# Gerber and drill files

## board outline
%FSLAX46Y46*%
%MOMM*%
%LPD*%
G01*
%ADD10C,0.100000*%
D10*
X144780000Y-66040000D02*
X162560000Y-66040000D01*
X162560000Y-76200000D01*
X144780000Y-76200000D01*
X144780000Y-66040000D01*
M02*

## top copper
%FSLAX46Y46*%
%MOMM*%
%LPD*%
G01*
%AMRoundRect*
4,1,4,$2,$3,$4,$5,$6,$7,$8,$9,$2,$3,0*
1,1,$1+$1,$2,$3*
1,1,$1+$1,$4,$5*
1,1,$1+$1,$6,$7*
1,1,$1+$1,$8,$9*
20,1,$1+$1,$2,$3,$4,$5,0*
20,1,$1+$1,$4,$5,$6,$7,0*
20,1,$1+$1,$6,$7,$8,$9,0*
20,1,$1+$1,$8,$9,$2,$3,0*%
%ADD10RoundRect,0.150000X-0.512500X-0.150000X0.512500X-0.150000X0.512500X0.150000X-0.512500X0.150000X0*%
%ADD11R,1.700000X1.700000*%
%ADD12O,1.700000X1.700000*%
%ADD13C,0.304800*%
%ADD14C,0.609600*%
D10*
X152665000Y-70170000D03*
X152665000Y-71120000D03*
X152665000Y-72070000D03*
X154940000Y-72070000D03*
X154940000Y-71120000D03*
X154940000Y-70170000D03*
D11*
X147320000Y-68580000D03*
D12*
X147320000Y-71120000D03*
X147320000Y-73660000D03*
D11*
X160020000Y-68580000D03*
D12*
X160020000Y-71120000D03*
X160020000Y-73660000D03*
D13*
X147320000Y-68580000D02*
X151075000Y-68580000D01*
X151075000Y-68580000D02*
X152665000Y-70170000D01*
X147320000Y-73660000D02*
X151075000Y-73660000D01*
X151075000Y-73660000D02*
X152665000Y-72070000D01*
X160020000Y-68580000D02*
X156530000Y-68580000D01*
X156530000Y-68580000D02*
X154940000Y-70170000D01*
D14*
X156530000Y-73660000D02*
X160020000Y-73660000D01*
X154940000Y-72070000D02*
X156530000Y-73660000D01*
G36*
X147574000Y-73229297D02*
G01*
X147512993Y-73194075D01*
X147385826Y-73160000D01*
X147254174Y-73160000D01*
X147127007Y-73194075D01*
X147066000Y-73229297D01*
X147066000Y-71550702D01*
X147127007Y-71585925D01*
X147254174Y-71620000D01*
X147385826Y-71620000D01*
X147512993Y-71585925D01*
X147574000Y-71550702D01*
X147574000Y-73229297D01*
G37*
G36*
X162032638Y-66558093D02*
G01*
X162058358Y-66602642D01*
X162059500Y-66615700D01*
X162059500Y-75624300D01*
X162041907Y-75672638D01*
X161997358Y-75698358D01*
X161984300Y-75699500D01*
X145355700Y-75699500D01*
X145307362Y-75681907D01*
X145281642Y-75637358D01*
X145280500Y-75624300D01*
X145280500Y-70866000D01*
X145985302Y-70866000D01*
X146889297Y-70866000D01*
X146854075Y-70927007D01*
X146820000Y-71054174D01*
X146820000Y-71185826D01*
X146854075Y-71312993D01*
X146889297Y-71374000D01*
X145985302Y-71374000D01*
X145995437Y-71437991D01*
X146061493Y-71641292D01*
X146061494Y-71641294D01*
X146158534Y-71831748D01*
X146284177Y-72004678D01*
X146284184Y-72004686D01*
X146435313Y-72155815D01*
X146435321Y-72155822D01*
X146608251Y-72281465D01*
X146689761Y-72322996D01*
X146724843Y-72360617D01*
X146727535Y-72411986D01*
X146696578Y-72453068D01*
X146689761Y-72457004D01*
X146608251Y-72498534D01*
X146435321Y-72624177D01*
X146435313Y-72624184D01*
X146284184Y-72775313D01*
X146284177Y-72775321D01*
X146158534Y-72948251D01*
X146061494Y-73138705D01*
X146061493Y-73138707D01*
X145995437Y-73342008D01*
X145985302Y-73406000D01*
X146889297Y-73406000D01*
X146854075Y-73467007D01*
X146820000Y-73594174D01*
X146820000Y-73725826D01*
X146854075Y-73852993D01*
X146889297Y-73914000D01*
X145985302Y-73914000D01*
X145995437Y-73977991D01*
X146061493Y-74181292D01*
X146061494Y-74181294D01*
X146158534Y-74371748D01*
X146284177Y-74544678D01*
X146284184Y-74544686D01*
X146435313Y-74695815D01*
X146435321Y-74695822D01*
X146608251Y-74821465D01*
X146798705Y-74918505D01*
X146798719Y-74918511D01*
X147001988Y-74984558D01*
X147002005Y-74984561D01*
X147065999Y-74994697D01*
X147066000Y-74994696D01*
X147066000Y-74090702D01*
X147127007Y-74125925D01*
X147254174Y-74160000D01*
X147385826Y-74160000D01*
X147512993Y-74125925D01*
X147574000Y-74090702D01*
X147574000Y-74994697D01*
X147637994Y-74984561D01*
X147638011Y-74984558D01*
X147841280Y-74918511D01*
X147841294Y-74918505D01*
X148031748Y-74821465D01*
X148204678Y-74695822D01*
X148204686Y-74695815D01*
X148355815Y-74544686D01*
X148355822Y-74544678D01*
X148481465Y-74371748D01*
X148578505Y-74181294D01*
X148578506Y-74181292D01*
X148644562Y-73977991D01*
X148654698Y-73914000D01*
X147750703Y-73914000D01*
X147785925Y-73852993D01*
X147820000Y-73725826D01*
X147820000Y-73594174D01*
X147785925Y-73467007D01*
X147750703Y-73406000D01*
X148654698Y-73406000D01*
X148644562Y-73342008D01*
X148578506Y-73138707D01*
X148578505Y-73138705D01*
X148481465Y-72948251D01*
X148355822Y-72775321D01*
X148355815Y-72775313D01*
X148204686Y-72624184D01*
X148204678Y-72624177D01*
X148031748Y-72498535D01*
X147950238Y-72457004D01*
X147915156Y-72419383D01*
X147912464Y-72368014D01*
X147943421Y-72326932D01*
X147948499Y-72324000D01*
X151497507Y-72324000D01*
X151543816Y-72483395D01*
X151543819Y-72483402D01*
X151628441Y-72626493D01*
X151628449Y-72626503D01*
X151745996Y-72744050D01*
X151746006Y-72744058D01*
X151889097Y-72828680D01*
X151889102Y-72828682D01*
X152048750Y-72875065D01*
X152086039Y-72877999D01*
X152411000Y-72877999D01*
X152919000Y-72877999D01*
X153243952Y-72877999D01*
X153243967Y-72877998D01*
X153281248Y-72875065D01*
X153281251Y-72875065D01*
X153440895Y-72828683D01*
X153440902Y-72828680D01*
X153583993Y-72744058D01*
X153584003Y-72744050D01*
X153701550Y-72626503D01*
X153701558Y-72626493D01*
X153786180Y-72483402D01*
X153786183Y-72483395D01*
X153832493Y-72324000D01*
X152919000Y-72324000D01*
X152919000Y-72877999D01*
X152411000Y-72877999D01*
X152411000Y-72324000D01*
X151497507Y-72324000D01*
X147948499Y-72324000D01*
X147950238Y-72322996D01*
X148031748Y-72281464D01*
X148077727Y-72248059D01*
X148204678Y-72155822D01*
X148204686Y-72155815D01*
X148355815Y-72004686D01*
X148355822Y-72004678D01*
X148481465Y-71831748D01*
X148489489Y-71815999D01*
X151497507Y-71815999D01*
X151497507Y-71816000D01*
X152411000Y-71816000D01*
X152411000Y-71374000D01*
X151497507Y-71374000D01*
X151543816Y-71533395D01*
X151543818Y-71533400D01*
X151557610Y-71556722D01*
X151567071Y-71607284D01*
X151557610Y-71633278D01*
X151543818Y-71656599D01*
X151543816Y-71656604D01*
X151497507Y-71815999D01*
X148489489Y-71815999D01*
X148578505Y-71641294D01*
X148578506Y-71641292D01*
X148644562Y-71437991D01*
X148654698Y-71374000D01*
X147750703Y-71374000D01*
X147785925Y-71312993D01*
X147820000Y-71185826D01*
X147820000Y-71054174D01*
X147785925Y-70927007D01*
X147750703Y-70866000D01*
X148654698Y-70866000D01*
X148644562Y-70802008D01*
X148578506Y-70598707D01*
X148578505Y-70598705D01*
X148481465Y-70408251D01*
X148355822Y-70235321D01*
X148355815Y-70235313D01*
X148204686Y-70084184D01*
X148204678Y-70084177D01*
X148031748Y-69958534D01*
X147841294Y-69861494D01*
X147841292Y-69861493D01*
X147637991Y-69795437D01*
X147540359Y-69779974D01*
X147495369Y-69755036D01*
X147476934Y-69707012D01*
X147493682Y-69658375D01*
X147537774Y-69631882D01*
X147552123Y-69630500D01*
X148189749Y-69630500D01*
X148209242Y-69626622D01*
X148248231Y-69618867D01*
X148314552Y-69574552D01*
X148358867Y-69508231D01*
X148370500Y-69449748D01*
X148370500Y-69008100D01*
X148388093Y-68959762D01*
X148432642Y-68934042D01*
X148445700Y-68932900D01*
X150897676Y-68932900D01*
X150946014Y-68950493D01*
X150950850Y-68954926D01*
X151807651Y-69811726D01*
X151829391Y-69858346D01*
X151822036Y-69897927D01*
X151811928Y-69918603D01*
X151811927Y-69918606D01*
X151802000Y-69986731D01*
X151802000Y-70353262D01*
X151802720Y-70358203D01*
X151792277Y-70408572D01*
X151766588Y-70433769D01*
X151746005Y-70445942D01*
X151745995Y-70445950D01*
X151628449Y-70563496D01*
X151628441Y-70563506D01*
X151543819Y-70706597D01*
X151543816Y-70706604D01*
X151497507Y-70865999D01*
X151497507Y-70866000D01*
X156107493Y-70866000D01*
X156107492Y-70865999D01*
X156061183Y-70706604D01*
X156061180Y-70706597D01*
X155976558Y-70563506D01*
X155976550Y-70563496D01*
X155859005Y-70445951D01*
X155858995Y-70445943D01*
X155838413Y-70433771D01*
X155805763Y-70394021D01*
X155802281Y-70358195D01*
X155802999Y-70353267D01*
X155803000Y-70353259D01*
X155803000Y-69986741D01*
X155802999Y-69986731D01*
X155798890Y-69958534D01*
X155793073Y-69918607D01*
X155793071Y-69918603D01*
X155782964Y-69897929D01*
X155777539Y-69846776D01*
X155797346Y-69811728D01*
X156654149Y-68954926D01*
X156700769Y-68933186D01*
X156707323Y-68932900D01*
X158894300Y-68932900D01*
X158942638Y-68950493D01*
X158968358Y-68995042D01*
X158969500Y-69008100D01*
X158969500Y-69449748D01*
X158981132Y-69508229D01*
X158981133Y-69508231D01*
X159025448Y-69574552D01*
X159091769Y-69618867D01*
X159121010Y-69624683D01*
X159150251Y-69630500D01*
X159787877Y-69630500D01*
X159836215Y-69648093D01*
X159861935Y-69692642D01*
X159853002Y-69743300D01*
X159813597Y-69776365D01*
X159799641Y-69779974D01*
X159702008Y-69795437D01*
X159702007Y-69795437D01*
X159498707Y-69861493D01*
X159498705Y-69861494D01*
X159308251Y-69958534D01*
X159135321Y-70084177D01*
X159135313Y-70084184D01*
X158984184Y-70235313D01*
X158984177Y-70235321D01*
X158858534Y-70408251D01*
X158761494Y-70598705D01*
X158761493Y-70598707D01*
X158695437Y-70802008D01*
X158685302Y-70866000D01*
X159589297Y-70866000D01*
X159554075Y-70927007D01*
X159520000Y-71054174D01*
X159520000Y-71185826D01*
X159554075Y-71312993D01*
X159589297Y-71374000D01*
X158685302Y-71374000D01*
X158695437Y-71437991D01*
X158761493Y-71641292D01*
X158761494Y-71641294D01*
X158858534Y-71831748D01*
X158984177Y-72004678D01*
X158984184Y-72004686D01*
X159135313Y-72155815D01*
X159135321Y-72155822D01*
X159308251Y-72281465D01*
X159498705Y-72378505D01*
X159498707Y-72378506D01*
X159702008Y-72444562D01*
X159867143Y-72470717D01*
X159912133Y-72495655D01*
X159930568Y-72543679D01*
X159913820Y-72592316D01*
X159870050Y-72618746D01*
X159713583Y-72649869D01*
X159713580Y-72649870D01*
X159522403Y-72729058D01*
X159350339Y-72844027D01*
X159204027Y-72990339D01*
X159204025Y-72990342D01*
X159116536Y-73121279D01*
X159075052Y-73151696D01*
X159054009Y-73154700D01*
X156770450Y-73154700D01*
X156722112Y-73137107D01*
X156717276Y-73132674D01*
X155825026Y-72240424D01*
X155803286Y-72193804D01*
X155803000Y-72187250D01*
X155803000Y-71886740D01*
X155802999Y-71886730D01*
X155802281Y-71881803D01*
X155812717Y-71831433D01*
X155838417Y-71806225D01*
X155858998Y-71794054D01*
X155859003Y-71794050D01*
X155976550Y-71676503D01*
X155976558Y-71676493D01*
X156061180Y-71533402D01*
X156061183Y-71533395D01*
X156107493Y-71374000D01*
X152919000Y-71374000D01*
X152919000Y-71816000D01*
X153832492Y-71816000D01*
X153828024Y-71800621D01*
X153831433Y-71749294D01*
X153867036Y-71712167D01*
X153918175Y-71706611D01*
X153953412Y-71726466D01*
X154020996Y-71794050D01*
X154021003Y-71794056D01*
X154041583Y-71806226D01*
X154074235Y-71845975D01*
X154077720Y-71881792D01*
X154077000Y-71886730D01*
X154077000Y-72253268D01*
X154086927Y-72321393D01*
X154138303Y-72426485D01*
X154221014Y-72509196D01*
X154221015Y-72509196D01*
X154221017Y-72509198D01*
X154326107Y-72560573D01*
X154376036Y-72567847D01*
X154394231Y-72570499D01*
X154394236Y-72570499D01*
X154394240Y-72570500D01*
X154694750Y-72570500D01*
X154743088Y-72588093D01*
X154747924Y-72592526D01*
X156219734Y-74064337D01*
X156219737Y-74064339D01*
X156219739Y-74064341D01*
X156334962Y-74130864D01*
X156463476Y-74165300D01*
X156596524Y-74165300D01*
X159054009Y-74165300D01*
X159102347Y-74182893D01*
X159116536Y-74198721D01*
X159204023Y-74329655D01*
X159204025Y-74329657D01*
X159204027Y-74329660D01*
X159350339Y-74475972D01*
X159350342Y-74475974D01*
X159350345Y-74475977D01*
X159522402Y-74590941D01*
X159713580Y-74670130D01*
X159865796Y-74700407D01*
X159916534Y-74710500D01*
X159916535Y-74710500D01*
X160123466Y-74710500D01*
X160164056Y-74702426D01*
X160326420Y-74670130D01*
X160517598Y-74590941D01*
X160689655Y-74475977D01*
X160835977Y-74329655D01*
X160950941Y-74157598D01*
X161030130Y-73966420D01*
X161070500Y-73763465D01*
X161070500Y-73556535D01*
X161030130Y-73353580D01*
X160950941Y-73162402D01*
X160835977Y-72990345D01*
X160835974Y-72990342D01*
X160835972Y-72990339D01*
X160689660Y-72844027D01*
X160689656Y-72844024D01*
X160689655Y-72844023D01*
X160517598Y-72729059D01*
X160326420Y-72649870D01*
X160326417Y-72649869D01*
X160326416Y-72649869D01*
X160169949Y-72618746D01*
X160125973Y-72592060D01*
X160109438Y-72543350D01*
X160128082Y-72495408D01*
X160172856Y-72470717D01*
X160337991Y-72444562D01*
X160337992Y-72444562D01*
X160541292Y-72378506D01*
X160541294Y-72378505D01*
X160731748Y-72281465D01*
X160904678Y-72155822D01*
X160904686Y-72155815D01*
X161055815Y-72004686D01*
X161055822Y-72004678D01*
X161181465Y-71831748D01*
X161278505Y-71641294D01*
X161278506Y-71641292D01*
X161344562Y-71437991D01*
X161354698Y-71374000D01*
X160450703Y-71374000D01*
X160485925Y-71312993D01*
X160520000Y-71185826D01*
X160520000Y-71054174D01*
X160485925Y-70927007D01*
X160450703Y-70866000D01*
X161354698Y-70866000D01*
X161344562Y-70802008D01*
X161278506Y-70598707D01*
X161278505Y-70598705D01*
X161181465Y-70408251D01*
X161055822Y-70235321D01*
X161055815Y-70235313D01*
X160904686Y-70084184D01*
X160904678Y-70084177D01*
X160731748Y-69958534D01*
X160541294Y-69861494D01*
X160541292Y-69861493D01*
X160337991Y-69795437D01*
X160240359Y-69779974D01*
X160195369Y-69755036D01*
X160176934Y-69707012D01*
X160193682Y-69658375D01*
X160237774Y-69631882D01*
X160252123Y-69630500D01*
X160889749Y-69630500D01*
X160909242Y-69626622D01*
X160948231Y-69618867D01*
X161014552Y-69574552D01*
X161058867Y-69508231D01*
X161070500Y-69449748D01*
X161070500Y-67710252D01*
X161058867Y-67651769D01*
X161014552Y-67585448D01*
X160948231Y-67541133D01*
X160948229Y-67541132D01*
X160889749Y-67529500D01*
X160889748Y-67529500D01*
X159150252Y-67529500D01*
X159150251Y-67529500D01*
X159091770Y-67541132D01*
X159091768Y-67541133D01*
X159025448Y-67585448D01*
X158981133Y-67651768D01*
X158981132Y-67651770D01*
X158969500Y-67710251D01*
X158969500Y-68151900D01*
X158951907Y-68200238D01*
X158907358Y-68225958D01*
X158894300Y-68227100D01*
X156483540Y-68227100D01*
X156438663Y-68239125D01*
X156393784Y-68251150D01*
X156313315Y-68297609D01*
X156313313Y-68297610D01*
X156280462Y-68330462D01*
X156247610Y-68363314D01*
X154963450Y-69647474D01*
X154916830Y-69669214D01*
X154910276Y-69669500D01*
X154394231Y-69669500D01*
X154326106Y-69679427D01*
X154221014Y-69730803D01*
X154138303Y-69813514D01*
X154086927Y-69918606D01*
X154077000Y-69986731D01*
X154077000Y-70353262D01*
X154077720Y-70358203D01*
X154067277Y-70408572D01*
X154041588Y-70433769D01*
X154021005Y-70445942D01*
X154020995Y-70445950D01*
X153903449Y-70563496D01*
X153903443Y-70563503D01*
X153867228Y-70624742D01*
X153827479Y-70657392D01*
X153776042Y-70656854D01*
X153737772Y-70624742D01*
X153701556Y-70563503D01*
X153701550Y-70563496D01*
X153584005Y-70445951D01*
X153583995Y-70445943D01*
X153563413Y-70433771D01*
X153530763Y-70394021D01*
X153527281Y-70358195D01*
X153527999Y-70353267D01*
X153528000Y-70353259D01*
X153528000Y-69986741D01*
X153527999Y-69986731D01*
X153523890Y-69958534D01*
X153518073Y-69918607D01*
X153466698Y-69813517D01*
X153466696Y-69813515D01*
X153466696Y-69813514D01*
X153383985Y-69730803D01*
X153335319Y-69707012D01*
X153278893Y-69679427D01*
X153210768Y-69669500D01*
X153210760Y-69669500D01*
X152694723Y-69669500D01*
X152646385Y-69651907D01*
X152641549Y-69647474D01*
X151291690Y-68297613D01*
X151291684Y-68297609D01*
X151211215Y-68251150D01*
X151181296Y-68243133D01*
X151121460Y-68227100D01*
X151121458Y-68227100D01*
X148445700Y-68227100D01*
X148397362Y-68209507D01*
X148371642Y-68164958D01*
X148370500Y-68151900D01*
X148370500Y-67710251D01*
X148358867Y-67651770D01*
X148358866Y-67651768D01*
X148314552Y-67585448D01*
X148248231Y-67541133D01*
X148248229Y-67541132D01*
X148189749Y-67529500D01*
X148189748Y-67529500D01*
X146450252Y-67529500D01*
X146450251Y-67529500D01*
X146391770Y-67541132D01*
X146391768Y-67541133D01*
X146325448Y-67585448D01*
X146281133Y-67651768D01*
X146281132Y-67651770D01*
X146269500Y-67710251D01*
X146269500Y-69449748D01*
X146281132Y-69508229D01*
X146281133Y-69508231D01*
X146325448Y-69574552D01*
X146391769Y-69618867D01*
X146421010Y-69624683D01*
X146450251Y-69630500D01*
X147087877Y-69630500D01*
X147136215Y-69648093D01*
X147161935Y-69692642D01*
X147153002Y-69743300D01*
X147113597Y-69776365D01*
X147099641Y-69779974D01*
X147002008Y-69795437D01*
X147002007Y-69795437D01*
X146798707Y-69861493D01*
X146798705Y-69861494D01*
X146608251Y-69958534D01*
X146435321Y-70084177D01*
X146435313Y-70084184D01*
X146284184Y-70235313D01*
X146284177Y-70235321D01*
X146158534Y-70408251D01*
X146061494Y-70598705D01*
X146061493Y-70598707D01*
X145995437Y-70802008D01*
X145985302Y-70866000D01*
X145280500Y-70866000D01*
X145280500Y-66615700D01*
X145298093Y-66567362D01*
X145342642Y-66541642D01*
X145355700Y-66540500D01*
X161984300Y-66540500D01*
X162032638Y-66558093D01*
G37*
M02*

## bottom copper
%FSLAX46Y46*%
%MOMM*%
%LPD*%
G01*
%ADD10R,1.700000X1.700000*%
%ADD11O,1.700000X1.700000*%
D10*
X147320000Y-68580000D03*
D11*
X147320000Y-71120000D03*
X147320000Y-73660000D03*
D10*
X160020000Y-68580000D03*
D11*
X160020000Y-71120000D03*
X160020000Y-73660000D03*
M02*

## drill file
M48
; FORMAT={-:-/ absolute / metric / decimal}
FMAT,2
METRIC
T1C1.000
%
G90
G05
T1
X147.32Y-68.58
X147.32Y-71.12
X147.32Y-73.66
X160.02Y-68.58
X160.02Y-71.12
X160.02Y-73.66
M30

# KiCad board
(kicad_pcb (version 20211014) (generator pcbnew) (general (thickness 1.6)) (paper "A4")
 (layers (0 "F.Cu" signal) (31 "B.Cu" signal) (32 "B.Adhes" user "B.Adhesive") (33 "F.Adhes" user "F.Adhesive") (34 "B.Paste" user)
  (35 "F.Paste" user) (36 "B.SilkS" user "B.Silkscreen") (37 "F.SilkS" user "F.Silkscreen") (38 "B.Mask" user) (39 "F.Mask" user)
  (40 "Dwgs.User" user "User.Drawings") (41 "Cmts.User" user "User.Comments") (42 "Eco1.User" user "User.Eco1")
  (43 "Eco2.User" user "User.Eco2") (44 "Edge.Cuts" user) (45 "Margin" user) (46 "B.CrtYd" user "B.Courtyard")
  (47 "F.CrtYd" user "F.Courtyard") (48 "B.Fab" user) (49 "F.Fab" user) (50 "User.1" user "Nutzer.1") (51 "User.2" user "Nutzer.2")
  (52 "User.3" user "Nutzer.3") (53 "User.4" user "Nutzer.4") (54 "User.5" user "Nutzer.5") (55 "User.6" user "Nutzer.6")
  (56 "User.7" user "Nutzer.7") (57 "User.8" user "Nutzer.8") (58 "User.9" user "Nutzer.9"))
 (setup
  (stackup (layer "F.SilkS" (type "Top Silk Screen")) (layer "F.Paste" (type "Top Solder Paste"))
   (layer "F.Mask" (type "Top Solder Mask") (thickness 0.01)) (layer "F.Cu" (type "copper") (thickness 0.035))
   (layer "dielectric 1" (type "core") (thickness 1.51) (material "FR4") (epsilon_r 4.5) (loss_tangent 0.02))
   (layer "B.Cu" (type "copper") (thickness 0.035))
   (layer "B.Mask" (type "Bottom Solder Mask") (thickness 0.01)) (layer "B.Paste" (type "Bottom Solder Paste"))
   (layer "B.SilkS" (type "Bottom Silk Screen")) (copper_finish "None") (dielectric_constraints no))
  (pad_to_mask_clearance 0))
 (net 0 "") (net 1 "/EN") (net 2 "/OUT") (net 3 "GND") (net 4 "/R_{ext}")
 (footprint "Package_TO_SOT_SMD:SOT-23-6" (layer "F.Cu") (at 153.8025 71.12)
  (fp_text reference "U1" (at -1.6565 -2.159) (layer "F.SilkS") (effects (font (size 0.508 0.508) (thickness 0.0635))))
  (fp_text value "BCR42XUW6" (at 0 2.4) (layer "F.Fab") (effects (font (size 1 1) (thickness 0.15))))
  (pad "1" smd roundrect (at -1.1375 -0.95) (size 1.325 0.6) (layers "F.Cu" "F.Paste" "F.Mask") (roundrect_rratio 0.25) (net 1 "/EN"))
  (pad "2" smd roundrect (at -1.1375 0) (size 1.325 0.6) (layers "F.Cu" "F.Paste" "F.Mask") (roundrect_rratio 0.25) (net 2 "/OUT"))
  (pad "3" smd roundrect (at -1.1375 0.95) (size 1.325 0.6) (layers "F.Cu" "F.Paste" "F.Mask") (roundrect_rratio 0.25) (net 2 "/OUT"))
  (pad "4" smd roundrect (at 1.1375 0.95) (size 1.325 0.6) (layers "F.Cu" "F.Paste" "F.Mask") (roundrect_rratio 0.25) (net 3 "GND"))
  (pad "5" smd roundrect (at 1.1375 0) (size 1.325 0.6) (layers "F.Cu" "F.Paste" "F.Mask") (roundrect_rratio 0.25) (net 2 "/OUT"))
  (pad "6" smd roundrect (at 1.1375 -0.95) (size 1.325 0.6) (layers "F.Cu" "F.Paste" "F.Mask") (roundrect_rratio 0.25) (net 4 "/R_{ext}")))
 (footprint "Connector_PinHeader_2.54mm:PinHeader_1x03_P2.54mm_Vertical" (layer "B.Cu") (at 147.32 68.58 180)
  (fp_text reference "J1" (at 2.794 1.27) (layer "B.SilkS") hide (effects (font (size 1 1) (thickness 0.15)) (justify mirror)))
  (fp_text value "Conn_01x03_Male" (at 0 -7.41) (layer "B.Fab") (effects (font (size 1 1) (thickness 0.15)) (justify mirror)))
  (pad "1" thru_hole rect (at 0 0 180) (size 1.7 1.7) (drill 1) (layers *.Cu *.Mask) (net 1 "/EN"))
  (pad "2" thru_hole oval (at 0 -2.54 180) (size 1.7 1.7) (drill 1) (layers *.Cu *.Mask) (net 2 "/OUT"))
  (pad "3" thru_hole oval (at 0 -5.08 180) (size 1.7 1.7) (drill 1) (layers *.Cu *.Mask) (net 2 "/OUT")))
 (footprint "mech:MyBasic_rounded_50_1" (layer "B.Cu") (at 153.8025 71.12 180) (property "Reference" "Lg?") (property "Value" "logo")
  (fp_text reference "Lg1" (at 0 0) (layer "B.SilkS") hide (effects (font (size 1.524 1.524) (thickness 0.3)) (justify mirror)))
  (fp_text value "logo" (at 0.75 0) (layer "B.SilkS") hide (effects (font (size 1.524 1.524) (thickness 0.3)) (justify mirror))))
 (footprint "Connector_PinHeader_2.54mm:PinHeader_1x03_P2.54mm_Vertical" (layer "B.Cu") (at 160.02 68.58 180)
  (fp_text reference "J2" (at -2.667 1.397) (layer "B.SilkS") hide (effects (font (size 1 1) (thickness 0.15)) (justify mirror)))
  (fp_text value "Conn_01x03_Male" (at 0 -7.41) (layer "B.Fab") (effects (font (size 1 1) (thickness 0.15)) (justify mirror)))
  (pad "1" thru_hole rect (at 0 0 180) (size 1.7 1.7) (drill 1) (layers *.Cu *.Mask) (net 4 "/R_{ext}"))
  (pad "2" thru_hole oval (at 0 -2.54 180) (size 1.7 1.7) (drill 1) (layers *.Cu *.Mask) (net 2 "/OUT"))
  (pad "3" thru_hole oval (at 0 -5.08 180) (size 1.7 1.7) (drill 1) (layers *.Cu *.Mask) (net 3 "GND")))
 (gr_rect (start 144.78 66.04) (end 162.56 76.2) (layer "Edge.Cuts") (width 0.1) (fill none))
 (segment (start 147.32 68.58) (end 151.075 68.58) (width 0.3048) (layer "F.Cu") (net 1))
 (segment (start 151.075 68.58) (end 152.665 70.17) (width 0.3048) (layer "F.Cu") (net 1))
 (segment (start 147.32 73.66) (end 151.075 73.66) (width 0.3048) (layer "F.Cu") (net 2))
 (segment (start 151.075 73.66) (end 152.665 72.07) (width 0.3048) (layer "F.Cu") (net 2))
 (segment (start 160.02 68.58) (end 156.53 68.58) (width 0.3048) (layer "F.Cu") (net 4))
 (segment (start 156.53 68.58) (end 154.94 70.17) (width 0.3048) (layer "F.Cu") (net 4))
 (segment (start 156.53 73.66) (end 160.02 73.66) (width 0.6096) (layer "F.Cu") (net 3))
 (segment (start 154.94 72.07) (end 156.53 73.66) (width 0.6096) (layer "F.Cu") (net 3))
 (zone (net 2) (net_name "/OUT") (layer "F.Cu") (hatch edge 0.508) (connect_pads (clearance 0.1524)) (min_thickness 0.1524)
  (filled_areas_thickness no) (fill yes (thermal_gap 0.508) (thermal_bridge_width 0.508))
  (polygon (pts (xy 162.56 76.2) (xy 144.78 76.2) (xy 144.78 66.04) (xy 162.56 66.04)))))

